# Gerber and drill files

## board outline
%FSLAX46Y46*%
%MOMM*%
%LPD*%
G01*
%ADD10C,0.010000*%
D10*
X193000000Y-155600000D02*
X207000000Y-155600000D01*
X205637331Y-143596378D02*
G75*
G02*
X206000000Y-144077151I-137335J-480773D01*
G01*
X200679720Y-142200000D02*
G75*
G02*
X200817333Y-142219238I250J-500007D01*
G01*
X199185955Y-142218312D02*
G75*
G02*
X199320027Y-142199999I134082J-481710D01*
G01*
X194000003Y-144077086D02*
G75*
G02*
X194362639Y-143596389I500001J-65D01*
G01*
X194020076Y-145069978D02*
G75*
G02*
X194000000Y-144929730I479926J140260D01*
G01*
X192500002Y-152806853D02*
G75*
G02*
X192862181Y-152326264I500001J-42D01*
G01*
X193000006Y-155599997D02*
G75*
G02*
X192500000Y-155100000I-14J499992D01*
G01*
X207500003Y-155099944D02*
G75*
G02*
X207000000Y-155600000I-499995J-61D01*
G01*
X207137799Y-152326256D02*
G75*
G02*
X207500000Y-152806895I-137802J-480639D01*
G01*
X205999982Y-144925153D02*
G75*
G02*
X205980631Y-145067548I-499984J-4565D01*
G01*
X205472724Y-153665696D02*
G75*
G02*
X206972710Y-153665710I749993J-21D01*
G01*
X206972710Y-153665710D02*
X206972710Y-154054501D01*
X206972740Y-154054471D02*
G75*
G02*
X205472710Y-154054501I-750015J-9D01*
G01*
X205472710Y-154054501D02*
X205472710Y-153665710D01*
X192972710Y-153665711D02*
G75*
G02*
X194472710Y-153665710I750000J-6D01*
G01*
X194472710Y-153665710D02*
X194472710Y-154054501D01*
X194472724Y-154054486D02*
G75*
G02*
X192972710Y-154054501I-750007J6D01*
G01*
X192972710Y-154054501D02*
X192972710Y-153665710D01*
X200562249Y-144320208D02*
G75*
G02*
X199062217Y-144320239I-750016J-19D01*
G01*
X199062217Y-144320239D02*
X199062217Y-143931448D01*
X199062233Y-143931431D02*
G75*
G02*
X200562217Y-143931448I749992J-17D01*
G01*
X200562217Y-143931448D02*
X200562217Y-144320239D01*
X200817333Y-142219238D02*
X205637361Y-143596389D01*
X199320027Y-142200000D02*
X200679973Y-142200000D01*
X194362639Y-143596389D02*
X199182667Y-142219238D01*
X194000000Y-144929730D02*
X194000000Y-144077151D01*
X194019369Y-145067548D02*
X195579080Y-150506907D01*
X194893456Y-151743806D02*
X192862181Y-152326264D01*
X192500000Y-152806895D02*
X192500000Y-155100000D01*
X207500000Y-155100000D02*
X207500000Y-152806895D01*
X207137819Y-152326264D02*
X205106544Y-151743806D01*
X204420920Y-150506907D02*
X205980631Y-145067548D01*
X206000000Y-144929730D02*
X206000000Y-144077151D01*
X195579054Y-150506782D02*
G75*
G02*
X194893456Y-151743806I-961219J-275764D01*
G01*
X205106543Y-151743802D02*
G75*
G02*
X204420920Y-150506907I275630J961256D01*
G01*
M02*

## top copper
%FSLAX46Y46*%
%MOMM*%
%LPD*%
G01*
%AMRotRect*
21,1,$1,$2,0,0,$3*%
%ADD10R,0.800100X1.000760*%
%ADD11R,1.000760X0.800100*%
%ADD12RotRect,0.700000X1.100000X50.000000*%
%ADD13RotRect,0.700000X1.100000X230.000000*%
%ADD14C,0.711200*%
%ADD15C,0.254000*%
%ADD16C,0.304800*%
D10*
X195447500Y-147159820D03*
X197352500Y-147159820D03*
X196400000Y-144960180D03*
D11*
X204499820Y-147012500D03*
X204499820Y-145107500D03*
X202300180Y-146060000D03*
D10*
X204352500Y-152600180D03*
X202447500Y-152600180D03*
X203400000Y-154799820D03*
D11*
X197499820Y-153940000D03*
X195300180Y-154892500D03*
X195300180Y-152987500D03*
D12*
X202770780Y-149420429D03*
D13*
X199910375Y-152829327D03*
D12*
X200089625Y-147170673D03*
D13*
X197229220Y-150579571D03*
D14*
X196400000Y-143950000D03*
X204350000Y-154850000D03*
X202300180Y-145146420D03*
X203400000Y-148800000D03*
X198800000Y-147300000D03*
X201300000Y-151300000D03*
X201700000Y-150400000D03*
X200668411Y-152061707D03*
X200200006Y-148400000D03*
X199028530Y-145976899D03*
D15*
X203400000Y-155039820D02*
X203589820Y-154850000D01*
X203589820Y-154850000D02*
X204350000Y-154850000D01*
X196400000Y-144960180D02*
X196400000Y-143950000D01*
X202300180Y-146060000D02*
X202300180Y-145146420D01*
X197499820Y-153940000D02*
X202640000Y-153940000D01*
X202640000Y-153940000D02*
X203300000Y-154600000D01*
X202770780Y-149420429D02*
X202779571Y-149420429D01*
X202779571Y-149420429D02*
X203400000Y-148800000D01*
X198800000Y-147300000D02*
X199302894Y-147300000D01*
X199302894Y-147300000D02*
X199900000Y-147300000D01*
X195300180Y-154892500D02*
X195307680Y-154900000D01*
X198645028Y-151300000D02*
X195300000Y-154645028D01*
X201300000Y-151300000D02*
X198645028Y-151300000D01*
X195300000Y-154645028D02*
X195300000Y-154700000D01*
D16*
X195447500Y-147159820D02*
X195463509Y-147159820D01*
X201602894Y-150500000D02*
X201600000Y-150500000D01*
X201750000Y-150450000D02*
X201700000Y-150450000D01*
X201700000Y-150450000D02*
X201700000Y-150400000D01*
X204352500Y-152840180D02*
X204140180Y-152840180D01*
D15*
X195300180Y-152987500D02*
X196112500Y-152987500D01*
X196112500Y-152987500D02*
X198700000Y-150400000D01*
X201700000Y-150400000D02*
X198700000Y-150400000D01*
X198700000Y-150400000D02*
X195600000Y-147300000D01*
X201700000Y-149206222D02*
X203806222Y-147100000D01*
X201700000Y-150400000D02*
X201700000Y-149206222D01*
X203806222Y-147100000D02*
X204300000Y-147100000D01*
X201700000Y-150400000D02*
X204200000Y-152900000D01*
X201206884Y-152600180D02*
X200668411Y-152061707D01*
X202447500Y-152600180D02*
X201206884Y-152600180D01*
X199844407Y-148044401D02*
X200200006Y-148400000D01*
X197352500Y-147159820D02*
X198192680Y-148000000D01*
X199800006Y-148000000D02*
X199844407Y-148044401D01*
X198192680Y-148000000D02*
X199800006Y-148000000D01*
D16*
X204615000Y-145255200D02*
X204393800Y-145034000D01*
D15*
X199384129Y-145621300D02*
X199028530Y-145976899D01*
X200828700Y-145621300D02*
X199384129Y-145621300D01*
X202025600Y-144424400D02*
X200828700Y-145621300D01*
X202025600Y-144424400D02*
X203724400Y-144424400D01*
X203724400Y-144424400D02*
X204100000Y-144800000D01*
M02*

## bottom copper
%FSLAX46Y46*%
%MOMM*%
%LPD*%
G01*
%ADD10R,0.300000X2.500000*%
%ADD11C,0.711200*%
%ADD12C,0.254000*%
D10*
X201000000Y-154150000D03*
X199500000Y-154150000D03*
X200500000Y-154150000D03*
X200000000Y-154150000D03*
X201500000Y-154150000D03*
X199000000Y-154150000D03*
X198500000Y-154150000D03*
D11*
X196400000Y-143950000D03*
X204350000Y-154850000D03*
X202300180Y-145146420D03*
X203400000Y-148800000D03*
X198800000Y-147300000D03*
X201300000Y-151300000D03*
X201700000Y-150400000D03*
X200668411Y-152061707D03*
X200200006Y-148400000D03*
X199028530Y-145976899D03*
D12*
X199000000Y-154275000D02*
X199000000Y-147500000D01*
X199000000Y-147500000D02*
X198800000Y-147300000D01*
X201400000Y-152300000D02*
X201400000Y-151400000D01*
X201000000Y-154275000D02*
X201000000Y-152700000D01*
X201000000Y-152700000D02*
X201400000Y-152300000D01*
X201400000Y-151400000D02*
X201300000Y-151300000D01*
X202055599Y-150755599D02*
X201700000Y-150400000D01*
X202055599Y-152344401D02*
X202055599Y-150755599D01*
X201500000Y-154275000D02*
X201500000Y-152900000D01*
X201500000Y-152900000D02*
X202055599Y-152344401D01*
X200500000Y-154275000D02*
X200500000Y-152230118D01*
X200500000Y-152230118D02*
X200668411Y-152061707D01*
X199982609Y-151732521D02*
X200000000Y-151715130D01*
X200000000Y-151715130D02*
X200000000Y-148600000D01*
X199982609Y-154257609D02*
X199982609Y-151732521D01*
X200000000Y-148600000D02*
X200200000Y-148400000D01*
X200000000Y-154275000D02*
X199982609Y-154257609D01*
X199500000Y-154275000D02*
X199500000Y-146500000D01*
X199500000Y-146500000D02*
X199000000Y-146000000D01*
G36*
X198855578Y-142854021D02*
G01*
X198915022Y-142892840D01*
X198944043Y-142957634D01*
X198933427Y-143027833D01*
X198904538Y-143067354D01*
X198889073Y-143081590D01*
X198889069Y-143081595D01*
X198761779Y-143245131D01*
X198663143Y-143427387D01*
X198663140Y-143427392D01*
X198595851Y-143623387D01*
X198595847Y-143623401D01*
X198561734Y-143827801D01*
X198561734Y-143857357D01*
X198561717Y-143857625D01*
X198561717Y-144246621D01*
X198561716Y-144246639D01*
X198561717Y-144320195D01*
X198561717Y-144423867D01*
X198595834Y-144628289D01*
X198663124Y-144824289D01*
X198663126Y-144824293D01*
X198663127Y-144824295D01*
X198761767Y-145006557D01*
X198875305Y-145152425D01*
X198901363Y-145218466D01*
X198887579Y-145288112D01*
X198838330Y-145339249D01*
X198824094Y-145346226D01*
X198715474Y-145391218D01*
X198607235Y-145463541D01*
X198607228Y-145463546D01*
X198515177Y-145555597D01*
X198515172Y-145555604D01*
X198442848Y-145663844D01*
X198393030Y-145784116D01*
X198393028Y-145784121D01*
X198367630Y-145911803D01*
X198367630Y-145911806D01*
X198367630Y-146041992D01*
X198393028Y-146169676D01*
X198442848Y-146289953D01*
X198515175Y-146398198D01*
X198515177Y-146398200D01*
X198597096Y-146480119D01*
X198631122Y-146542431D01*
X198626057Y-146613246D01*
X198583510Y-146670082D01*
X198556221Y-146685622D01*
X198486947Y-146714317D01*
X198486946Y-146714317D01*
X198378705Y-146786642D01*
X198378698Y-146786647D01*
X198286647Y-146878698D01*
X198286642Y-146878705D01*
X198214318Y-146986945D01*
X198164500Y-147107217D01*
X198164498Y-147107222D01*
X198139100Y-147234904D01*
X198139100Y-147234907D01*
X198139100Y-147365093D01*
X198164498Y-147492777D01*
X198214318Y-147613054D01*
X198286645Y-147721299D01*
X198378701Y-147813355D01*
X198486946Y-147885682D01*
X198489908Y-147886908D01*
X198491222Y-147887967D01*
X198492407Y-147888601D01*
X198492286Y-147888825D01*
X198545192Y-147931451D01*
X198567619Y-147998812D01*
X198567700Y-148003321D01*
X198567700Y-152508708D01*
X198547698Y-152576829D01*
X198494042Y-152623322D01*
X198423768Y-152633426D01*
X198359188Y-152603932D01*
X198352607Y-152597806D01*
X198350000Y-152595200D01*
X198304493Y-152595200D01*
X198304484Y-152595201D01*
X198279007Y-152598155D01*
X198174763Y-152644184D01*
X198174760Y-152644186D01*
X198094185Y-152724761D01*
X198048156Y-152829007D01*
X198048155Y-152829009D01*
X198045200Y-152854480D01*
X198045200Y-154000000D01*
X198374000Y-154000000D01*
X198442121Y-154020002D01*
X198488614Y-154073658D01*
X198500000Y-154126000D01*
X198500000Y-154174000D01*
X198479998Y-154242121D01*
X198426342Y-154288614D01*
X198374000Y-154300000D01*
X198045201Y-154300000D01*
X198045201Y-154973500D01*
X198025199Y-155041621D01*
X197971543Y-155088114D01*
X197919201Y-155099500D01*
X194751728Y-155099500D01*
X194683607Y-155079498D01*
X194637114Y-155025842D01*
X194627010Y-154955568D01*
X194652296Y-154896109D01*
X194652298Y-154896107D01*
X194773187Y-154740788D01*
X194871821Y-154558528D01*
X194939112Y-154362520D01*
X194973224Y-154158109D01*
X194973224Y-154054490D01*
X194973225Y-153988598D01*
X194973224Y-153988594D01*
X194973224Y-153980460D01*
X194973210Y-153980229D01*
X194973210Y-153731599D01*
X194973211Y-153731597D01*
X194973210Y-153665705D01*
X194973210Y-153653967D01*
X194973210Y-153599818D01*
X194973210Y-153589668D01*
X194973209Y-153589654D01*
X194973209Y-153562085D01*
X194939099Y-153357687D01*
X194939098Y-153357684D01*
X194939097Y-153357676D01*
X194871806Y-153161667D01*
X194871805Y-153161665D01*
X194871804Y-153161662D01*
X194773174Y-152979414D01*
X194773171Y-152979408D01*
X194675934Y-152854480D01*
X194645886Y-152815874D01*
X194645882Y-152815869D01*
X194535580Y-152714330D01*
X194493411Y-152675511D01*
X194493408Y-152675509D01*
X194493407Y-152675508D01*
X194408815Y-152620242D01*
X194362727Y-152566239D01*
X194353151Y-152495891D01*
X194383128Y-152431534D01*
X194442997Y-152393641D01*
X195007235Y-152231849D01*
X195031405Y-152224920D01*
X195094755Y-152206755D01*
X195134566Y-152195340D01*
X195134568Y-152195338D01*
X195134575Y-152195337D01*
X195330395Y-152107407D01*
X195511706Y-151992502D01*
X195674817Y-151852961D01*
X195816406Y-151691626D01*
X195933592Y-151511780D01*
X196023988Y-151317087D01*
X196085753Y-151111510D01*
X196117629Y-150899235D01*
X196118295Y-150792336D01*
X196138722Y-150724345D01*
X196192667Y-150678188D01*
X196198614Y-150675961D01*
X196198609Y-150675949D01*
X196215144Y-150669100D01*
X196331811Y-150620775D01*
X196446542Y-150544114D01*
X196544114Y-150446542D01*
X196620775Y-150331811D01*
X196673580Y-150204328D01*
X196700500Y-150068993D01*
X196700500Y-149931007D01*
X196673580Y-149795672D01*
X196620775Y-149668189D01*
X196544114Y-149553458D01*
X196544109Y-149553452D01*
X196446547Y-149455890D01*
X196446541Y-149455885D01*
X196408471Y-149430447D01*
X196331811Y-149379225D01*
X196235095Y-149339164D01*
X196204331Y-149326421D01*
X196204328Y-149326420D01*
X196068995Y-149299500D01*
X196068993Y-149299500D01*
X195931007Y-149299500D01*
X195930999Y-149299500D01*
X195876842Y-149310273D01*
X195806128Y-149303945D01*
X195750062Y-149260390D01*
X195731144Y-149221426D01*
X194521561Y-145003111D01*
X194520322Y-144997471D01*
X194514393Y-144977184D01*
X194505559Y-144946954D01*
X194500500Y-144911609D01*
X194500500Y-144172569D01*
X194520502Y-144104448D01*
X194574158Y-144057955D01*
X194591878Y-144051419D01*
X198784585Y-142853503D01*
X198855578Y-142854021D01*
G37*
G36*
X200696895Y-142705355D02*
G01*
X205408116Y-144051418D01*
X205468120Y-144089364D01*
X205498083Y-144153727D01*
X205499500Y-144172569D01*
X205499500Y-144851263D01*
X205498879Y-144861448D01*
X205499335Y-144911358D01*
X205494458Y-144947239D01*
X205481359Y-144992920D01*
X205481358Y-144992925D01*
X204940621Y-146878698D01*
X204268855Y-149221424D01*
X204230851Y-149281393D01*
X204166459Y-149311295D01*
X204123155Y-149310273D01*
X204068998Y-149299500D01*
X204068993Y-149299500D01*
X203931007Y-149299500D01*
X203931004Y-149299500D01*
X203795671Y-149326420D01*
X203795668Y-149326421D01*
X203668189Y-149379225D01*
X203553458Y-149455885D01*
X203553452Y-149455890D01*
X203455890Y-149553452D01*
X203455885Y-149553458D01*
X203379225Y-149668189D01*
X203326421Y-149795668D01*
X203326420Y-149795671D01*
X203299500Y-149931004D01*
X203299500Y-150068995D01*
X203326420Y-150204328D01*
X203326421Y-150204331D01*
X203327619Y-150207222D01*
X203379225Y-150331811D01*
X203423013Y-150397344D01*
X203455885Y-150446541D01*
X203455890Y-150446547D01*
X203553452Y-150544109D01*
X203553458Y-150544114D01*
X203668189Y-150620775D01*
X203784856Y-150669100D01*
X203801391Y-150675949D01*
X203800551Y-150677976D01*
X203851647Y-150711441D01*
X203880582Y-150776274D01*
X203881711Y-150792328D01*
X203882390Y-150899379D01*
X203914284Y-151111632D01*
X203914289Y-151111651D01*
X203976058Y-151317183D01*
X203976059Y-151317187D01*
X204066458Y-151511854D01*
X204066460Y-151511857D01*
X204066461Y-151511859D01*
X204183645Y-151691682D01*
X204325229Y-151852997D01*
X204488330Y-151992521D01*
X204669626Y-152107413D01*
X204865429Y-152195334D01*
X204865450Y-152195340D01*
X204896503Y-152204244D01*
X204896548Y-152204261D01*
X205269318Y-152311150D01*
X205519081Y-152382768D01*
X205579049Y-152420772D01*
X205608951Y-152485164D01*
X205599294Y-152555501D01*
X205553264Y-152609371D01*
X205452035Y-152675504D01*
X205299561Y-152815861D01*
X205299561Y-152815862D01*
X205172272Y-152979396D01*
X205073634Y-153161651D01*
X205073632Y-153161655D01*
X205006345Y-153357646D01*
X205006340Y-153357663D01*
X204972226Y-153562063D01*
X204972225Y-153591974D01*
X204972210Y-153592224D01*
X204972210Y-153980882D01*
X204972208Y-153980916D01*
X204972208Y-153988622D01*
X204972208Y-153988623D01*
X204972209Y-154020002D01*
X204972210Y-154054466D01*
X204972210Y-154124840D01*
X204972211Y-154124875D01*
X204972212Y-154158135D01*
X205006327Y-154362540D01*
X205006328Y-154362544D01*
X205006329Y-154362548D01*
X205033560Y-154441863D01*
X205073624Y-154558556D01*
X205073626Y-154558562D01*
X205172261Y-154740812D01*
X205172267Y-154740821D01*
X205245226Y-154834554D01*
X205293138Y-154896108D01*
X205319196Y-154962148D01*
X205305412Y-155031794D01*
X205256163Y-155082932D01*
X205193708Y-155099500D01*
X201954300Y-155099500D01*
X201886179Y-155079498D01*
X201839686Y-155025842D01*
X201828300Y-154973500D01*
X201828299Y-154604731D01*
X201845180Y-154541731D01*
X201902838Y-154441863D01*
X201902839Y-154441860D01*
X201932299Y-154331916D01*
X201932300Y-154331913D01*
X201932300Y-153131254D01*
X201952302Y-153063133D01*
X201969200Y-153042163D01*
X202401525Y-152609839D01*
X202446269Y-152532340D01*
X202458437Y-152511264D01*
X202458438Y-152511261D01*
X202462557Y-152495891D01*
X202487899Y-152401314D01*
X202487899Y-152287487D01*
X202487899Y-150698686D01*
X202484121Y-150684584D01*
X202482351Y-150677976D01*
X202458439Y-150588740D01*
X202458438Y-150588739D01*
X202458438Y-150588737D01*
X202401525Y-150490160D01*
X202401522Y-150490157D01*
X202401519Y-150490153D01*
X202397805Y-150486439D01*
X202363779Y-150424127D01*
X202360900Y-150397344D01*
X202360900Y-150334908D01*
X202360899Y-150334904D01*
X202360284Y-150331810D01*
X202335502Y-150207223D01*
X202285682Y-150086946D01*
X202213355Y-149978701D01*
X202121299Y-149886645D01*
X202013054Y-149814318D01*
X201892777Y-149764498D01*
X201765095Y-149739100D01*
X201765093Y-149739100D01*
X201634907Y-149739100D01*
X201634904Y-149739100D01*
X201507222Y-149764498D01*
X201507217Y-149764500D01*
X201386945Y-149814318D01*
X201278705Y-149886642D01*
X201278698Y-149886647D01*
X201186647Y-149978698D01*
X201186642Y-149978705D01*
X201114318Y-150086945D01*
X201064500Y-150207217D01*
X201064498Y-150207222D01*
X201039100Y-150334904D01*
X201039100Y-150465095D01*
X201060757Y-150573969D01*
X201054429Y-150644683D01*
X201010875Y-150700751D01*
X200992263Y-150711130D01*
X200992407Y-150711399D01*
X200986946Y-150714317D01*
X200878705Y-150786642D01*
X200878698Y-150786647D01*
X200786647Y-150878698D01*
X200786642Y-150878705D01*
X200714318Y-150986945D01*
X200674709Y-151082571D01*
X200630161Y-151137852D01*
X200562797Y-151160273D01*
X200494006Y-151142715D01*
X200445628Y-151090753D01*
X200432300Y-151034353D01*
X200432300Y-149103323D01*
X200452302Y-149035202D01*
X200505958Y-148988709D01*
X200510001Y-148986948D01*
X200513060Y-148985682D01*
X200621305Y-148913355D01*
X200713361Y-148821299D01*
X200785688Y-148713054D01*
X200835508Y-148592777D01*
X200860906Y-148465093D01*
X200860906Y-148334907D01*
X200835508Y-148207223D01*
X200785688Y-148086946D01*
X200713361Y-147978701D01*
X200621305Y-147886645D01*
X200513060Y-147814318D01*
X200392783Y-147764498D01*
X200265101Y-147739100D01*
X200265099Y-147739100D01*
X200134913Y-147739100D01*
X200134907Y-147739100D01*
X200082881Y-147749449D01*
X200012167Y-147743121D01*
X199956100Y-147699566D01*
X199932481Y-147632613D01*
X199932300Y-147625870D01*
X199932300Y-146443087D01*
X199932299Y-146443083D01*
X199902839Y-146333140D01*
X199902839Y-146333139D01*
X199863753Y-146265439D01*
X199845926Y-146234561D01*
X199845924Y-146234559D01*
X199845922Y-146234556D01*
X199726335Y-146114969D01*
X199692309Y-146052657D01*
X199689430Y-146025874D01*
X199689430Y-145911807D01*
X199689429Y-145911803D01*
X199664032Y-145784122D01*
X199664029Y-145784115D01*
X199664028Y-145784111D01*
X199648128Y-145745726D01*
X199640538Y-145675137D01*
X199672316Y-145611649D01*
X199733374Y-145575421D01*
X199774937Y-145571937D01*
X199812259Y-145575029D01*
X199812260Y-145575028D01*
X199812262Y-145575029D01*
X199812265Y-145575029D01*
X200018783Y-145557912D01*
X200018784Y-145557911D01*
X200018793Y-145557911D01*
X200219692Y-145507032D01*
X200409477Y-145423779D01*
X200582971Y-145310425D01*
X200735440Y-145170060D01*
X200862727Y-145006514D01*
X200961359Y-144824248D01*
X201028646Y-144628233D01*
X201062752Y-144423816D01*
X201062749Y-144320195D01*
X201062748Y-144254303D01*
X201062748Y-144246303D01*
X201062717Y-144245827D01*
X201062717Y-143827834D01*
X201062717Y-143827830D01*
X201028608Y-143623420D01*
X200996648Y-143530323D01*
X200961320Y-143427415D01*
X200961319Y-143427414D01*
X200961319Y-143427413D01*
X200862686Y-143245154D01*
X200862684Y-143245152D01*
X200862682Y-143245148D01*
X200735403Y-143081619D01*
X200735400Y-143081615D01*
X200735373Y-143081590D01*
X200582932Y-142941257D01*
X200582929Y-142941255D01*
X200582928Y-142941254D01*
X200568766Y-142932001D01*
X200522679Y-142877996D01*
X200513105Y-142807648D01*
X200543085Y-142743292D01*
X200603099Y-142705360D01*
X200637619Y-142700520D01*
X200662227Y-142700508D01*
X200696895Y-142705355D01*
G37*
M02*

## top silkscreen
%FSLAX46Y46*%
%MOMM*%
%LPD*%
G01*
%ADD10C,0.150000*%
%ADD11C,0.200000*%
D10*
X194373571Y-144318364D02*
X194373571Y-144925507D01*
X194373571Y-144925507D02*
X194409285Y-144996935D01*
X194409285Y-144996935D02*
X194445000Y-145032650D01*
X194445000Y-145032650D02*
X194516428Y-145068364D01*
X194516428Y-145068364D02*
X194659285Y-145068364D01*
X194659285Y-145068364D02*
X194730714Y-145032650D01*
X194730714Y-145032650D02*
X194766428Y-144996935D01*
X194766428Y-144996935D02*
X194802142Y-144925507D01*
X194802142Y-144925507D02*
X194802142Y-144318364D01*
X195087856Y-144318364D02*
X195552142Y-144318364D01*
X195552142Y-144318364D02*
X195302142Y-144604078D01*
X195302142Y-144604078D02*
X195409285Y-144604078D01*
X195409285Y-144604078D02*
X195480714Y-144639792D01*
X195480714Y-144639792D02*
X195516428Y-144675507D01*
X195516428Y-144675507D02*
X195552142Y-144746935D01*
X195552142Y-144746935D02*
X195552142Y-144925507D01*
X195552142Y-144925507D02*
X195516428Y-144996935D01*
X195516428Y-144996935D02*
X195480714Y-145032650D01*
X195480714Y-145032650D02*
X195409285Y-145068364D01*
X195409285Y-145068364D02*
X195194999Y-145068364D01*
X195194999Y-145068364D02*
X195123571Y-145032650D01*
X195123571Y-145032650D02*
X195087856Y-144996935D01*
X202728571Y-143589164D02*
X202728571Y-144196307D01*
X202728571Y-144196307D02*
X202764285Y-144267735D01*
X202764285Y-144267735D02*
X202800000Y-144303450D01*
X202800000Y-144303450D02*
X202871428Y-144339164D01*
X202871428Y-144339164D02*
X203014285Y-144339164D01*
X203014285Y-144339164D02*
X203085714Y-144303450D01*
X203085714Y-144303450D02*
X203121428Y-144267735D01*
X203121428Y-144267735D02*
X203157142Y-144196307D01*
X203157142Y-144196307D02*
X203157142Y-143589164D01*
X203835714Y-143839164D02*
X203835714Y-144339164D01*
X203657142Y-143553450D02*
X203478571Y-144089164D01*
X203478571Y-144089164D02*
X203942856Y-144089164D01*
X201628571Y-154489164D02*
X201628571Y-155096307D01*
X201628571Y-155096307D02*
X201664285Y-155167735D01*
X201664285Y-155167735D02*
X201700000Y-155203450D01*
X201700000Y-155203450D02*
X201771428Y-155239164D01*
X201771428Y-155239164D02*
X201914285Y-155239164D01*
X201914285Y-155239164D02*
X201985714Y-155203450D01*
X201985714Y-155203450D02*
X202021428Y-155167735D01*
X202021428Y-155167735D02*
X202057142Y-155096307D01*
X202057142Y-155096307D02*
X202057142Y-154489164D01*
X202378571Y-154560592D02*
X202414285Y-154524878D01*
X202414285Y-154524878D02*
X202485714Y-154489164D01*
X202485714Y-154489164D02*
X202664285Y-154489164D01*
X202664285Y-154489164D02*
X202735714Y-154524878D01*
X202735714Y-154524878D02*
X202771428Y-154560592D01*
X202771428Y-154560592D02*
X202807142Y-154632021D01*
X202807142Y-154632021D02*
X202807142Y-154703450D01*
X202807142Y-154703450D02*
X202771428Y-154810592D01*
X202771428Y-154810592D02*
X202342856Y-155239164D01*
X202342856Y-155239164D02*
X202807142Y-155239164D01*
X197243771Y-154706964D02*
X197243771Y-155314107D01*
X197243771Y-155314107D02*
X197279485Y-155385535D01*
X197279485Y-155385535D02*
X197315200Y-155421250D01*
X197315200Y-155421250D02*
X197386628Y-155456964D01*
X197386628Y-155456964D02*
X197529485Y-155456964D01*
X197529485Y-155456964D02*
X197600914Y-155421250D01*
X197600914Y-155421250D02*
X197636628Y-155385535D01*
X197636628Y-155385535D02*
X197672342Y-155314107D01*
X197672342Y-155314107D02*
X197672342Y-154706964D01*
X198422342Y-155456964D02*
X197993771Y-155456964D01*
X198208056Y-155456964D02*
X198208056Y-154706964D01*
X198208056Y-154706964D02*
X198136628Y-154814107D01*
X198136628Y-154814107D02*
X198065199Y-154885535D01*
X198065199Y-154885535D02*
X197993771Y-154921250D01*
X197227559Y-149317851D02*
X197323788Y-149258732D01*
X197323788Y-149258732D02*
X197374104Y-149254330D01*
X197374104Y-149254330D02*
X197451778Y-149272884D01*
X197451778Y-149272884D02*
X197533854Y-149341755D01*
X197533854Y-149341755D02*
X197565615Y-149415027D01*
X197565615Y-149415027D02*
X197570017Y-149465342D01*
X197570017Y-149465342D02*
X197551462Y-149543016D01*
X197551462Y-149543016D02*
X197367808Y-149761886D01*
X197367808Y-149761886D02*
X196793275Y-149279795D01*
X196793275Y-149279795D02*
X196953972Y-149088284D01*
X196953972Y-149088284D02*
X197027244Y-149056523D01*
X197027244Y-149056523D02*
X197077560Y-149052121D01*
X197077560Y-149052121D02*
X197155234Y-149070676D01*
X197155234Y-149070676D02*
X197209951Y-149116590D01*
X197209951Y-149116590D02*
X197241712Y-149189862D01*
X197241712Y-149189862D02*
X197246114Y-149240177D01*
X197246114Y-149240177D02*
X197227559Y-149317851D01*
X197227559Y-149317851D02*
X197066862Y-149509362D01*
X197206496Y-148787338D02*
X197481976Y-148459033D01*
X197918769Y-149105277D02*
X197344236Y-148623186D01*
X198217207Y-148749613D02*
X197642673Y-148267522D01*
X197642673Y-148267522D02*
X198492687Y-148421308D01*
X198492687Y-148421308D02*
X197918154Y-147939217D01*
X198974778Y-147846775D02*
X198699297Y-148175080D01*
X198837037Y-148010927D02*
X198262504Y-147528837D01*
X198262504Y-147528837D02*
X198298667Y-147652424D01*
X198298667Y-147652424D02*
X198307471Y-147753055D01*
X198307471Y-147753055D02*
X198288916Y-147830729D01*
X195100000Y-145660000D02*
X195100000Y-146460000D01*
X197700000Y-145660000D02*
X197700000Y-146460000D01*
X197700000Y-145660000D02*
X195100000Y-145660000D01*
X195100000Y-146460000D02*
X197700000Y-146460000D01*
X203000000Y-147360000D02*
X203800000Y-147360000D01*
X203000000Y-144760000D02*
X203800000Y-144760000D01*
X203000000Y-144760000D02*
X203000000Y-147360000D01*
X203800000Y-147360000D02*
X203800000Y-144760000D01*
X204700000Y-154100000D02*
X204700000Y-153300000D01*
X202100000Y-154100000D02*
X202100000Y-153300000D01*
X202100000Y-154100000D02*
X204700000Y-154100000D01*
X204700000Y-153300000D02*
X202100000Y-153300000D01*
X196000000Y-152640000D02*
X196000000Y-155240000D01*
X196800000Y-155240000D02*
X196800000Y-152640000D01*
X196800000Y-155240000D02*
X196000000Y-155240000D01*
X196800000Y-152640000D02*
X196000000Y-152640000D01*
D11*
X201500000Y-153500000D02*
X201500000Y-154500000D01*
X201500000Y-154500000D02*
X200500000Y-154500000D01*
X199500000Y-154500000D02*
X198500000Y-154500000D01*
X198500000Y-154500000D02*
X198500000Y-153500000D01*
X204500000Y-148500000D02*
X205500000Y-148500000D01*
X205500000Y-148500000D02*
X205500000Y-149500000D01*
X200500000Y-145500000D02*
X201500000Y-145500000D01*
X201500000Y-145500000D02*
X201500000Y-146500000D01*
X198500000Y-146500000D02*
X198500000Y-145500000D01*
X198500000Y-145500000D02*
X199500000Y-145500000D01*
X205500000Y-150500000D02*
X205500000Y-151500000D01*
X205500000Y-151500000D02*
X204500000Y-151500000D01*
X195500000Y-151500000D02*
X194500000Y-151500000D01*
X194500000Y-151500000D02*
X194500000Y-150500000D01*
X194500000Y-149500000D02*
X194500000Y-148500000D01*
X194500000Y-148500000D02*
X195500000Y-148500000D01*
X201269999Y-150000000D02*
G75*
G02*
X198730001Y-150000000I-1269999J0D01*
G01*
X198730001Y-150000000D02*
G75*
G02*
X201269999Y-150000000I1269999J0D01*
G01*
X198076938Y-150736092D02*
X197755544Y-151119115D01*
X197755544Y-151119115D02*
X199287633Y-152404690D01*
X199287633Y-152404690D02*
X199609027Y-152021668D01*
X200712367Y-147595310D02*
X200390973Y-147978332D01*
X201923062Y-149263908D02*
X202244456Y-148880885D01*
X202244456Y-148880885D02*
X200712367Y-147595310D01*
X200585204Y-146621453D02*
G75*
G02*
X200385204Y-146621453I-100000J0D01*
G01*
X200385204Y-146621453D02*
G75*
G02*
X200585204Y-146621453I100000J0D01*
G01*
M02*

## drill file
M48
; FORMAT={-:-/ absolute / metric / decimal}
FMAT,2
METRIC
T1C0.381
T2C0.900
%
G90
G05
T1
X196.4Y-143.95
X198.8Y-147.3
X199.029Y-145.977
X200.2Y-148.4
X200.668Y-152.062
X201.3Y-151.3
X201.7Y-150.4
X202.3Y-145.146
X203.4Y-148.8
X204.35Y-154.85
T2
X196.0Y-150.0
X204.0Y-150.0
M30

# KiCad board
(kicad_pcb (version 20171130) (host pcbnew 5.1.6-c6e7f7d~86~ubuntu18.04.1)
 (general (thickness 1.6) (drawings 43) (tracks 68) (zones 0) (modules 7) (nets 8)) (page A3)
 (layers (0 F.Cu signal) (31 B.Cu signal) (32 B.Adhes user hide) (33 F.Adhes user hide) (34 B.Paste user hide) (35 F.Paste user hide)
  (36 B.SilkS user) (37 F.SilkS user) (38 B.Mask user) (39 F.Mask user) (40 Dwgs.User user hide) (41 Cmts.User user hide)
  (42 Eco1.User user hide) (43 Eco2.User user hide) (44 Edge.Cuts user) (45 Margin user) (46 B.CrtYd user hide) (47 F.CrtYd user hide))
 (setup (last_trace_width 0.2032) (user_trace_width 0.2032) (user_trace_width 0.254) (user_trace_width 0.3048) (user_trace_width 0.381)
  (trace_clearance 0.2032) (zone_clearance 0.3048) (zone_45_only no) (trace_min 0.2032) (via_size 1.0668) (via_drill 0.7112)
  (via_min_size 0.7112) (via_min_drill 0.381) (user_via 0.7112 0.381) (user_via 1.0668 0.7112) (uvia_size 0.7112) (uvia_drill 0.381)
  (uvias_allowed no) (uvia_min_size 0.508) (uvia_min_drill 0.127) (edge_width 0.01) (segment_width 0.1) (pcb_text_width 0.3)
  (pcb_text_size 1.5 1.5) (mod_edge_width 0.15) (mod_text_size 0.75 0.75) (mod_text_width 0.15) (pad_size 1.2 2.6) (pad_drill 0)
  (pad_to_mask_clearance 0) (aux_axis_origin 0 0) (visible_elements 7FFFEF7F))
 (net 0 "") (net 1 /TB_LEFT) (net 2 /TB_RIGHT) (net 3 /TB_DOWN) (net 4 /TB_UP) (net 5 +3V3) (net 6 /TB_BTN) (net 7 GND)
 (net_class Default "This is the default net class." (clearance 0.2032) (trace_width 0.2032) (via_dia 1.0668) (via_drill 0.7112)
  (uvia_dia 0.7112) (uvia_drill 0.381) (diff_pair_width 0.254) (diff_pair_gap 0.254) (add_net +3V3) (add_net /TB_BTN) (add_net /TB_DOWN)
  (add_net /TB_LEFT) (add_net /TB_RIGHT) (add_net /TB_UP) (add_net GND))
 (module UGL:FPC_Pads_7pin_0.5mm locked (layer B.Cu) (at 200 155.4 180)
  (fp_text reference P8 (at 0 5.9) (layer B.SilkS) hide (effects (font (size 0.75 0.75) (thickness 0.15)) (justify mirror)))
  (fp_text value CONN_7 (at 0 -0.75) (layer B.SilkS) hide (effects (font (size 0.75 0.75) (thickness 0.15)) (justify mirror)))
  (pad 2 smd rect (at -1 1.25 180) (size 0.3 2.5) (layers B.Cu B.Mask) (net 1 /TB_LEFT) (clearance 0.1778))
  (pad 5 smd rect (at 0.5 1.25 180) (size 0.3 2.5) (layers B.Cu B.Mask) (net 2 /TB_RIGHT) (clearance 0.1778))
  (pad 3 smd rect (at -0.5 1.25 180) (size 0.3 2.5) (layers B.Cu B.Mask) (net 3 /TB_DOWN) (clearance 0.1778))
  (pad 4 smd rect (at 0 1.25 180) (size 0.3 2.5) (layers B.Cu B.Mask) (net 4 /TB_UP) (clearance 0.1778))
  (pad 1 smd rect (at -1.5 1.25 180) (size 0.3 2.5) (layers B.Cu B.Mask) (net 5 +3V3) (clearance 0.1778))
  (pad 6 smd rect (at 1 1.25 180) (size 0.3 2.5) (layers B.Cu B.Mask) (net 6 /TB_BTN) (clearance 0.1778))
  (pad 7 smd rect (at 1.5 1.25 180) (size 0.3 2.5) (layers B.Cu B.Mask) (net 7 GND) (clearance 0.1778)))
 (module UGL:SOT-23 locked (layer F.Cu) (at 196.4 146.06)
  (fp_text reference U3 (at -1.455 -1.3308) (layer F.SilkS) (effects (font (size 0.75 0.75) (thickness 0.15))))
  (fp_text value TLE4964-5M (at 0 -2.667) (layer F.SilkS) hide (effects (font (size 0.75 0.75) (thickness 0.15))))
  (fp_line (start -1.3 -0.4) (end -1.3 0.4) (layer F.SilkS) (width 0.15))
  (fp_line (start 1.3 -0.4) (end 1.3 0.4) (layer F.SilkS) (width 0.15))
  (fp_line (start 1.3 -0.4) (end -1.3 -0.4) (layer F.SilkS) (width 0.15))
  (fp_line (start -1.3 0.4) (end 1.3 0.4) (layer F.SilkS) (width 0.15))
  (pad 1 smd rect (at -0.9525 1.09982) (size 0.8001 1.00076) (layers F.Cu F.Paste F.Mask) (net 5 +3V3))
  (pad 2 smd rect (at 0.9525 1.09982) (size 0.8001 1.00076) (layers F.Cu F.Paste F.Mask) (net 4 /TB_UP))
  (pad 3 smd rect (at 0 -1.09982) (size 0.8001 1.00076) (layers F.Cu F.Paste F.Mask) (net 7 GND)))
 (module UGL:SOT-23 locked (layer F.Cu) (at 203.4 146.06 90)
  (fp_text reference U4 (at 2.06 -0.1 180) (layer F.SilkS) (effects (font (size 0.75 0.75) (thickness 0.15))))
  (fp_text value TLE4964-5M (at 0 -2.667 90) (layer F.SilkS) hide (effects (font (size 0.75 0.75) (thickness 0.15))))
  (fp_line (start -1.3 -0.4) (end -1.3 0.4) (layer F.SilkS) (width 0.15))
  (fp_line (start 1.3 -0.4) (end 1.3 0.4) (layer F.SilkS) (width 0.15))
  (fp_line (start 1.3 -0.4) (end -1.3 -0.4) (layer F.SilkS) (width 0.15))
  (fp_line (start -1.3 0.4) (end 1.3 0.4) (layer F.SilkS) (width 0.15))
  (pad 1 smd rect (at -0.9525 1.09982 90) (size 0.8001 1.00076) (layers F.Cu F.Paste F.Mask) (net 5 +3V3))
  (pad 2 smd rect (at 0.9525 1.09982 90) (size 0.8001 1.00076) (layers F.Cu F.Paste F.Mask) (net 2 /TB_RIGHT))
  (pad 3 smd rect (at 0 -1.09982 90) (size 0.8001 1.00076) (layers F.Cu F.Paste F.Mask) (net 7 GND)))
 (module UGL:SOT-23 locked (layer F.Cu) (at 203.4 153.7 180)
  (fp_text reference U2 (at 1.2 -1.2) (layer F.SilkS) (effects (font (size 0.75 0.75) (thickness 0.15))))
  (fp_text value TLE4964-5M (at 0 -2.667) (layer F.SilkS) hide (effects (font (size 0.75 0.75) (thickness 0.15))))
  (fp_line (start -1.3 -0.4) (end -1.3 0.4) (layer F.SilkS) (width 0.15))
  (fp_line (start 1.3 -0.4) (end 1.3 0.4) (layer F.SilkS) (width 0.15))
  (fp_line (start 1.3 -0.4) (end -1.3 -0.4) (layer F.SilkS) (width 0.15))
  (fp_line (start -1.3 0.4) (end 1.3 0.4) (layer F.SilkS) (width 0.15))
  (pad 1 smd rect (at -0.9525 1.09982 180) (size 0.8001 1.00076) (layers F.Cu F.Paste F.Mask) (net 5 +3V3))
  (pad 2 smd rect (at 0.9525 1.09982 180) (size 0.8001 1.00076) (layers F.Cu F.Paste F.Mask) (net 3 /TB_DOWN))
  (pad 3 smd rect (at 0 -1.09982 180) (size 0.8001 1.00076) (layers F.Cu F.Paste F.Mask) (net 7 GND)))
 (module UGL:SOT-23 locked (layer F.Cu) (at 196.4 153.94 270)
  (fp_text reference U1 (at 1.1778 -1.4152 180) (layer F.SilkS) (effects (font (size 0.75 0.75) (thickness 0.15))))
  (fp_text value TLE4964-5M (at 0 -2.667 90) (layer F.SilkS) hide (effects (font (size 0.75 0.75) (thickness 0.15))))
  (fp_line (start -1.3 0.4) (end 1.3 0.4) (layer F.SilkS) (width 0.15))
  (fp_line (start 1.3 -0.4) (end -1.3 -0.4) (layer F.SilkS) (width 0.15))
  (fp_line (start 1.3 -0.4) (end 1.3 0.4) (layer F.SilkS) (width 0.15))
  (fp_line (start -1.3 -0.4) (end -1.3 0.4) (layer F.SilkS) (width 0.15))
  (pad 3 smd rect (at 0 -1.09982 270) (size 0.8001 1.00076) (layers F.Cu F.Paste F.Mask) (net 7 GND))
  (pad 2 smd rect (at 0.9525 1.09982 270) (size 0.8001 1.00076) (layers F.Cu F.Paste F.Mask) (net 1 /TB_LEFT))
  (pad 1 smd rect (at -0.9525 1.09982 270) (size 0.8001 1.00076) (layers F.Cu F.Paste F.Mask) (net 5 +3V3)))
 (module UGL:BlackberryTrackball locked (layer F.Cu) (at 200 150)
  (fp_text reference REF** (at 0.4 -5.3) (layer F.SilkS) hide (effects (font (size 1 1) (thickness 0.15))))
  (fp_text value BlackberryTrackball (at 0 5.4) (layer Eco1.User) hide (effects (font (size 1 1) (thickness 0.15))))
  (fp_line (start 1.5 3.5) (end 1.5 4.5) (layer F.SilkS) (width 0.2))
  (fp_line (start 1.5 4.5) (end 0.5 4.5) (layer F.SilkS) (width 0.2))
  (fp_line (start -0.5 4.5) (end -1.5 4.5) (layer F.SilkS) (width 0.2))
  (fp_line (start -1.5 4.5) (end -1.5 3.5) (layer F.SilkS) (width 0.2))
  (fp_line (start 4.5 -1.5) (end 5.5 -1.5) (layer F.SilkS) (width 0.2))
  (fp_line (start 5.5 -1.5) (end 5.5 -0.5) (layer F.SilkS) (width 0.2))
  (fp_line (start 0.5 -4.5) (end 1.5 -4.5) (layer F.SilkS) (width 0.2))
  (fp_line (start 1.5 -4.5) (end 1.5 -3.5) (layer F.SilkS) (width 0.2))
  (fp_line (start -1.5 -3.5) (end -1.5 -4.5) (layer F.SilkS) (width 0.2))
  (fp_line (start -1.5 -4.5) (end -0.5 -4.5) (layer F.SilkS) (width 0.2))
  (fp_line (start 5.5 0.5) (end 5.5 1.5) (layer F.SilkS) (width 0.2))
  (fp_line (start 5.5 1.5) (end 4.5 1.5) (layer F.SilkS) (width 0.2))
  (fp_line (start -4.5 1.5) (end -5.5 1.5) (layer F.SilkS) (width 0.2))
  (fp_line (start -5.5 1.5) (end -5.5 0.5) (layer F.SilkS) (width 0.2))
  (fp_line (start -5.5 -0.5) (end -5.5 -1.5) (layer F.SilkS) (width 0.2))
  (fp_line (start -5.5 -1.5) (end -4.5 -1.5) (layer F.SilkS) (width 0.2))
  (pad "" np_thru_hole circle (at 4 0) (size 0.9 0.9) (drill 0.9) (layers *.Cu *.Mask))
  (pad "" np_thru_hole circle (at -4 0) (size 0.9 0.9) (drill 0.9) (layers *.Cu *.Mask)))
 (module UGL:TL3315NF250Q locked (layer F.Cu) (at 200 150 50)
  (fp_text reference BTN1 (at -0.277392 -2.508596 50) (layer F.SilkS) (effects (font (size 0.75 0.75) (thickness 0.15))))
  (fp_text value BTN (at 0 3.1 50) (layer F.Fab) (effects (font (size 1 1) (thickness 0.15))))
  (fp_circle (center 0 0) (end 1.27 0) (layer F.SilkS) (width 0.2))
  (fp_line (start -1.8 -1) (end -2.3 -1) (layer F.SilkS) (width 0.2))
  (fp_line (start -2.3 -1) (end -2.3 1) (layer F.SilkS) (width 0.2))
  (fp_line (start -2.3 1) (end -1.8 1) (layer F.SilkS) (width 0.2))
  (fp_line (start 2.3 -1) (end 1.8 -1) (layer F.SilkS) (width 0.2))
  (fp_line (start 1.8 1) (end 2.3 1) (layer F.SilkS) (width 0.2))
  (fp_line (start 2.3 1) (end 2.3 -1) (layer F.SilkS) (width 0.2))
  (fp_circle (center 2.9 -1.8) (end 3 -1.8) (layer F.SilkS) (width 0.2))
  (pad 2 smd rect (at 2.225 1.75 50) (size 0.7 1.1) (layers F.Cu F.Paste F.Mask) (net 7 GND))
  (pad 3 smd rect (at -2.225 1.75 230) (size 0.7 1.1) (layers F.Cu F.Paste F.Mask))
  (pad 1 smd rect (at 2.225 -1.75 50) (size 0.7 1.1) (layers F.Cu F.Paste F.Mask) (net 6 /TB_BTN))
  (pad 4 smd rect (at -2.225 -1.75 230) (size 0.7 1.1) (layers F.Cu F.Paste F.Mask)))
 (gr_line (start 193 155.6) (end 207 155.6) (angle 90) (layer Edge.Cuts) (width 0.01))
 (gr_arc (start 205.499996 144.077151) (end 206 144.077151) (angle -74.05780781) (layer Edge.Cuts) (width 0.01))
 (gr_arc (start 200.67997 142.700007) (end 200.817333 142.219238) (angle -15.97405795) (layer Edge.Cuts) (width 0.01))
 (gr_arc (start 199.320037 142.700022) (end 199.320027 142.2) (angle -15.55315467) (layer Edge.Cuts) (width 0.01))
 (gr_arc (start 194.500004 144.077151) (end 194.362639 143.596389) (angle -74.04666612) (layer Edge.Cuts) (width 0.01))
 (gr_arc (start 194.500002 144.929718) (end 194 144.92973) (angle -16.28978266) (layer Edge.Cuts) (width 0.01))
 (gr_arc (start 193.000003 152.806895) (end 192.862181 152.326264) (angle -73.99483282) (layer Edge.Cuts) (width 0.01))
 (gr_arc (start 192.999992 155.100005) (end 192.5 155.1) (angle -90.00219193) (layer Edge.Cuts) (width 0.01))
 (gr_arc (start 207.000008 155.100005) (end 207 155.6) (angle -90.00795646) (layer Edge.Cuts) (width 0.01))
 (gr_arc (start 206.999997 152.806895) (end 207.5 152.806895) (angle -74.00205761) (layer Edge.Cuts) (width 0.01))
 (gr_arc (start 205.499998 144.929718) (end 205.980631 145.067548) (angle -16.5242857) (layer Edge.Cuts) (width 0.01))
 (gr_arc (start 206.222717 153.665717) (end 206.97271 153.66571) (angle -179.9978282) (layer Edge.Cuts) (width 0.01))
 (gr_line (start 206.97271 153.66571) (end 206.97271 154.054501) (angle 90) (layer Edge.Cuts) (width 0.01))
 (gr_arc (start 206.222725 154.05448) (end 205.47271 154.054501) (angle -179.9990721) (layer Edge.Cuts) (width 0.01))
 (gr_line (start 205.47271 154.054501) (end 205.47271 153.66571) (angle 90) (layer Edge.Cuts) (width 0.01))
 (gr_arc (start 193.72271 153.665717) (end 194.47271 153.66571) (angle -179.9989939) (layer Edge.Cuts) (width 0.01))
 (gr_line (start 194.47271 153.66571) (end 194.47271 154.054501) (angle 90) (layer Edge.Cuts) (width 0.01))
 (gr_arc (start 193.722717 154.05448) (end 192.97271 154.054501) (angle -179.9979064) (layer Edge.Cuts) (width 0.01))
 (gr_line (start 192.97271 154.054501) (end 192.97271 153.66571) (angle 90) (layer Edge.Cuts) (width 0.01))
 (gr_arc (start 199.812233 144.320227) (end 199.062217 144.320239) (angle -180.0005206) (layer Edge.Cuts) (width 0.01))
 (gr_line (start 199.062217 144.320239) (end 199.062217 143.931448) (angle 90) (layer Edge.Cuts) (width 0.01))
 (gr_arc (start 199.812225 143.931448) (end 200.562217 143.931448) (angle -179.9987111) (layer Edge.Cuts) (width 0.01))
 (gr_line (start 200.562217 143.931448) (end 200.562217 144.320239) (angle 90) (layer Edge.Cuts) (width 0.01))
 (gr_line (start 200.817333 142.219238) (end 205.637361 143.596389) (angle 90) (layer Edge.Cuts) (width 0.01))
 (gr_line (start 199.320027 142.2) (end 200.679973 142.2) (angle 90) (layer Edge.Cuts) (width 0.01))
 (gr_line (start 194.362639 143.596389) (end 199.182667 142.219238) (angle 90) (layer Edge.Cuts) (width 0.01))
 (gr_line (start 194 144.92973) (end 194 144.077151) (angle 90) (layer Edge.Cuts) (width 0.01))
 (gr_line (start 194.019369 145.067548) (end 195.57908 150.506907) (angle 90) (layer Edge.Cuts) (width 0.01))
 (gr_line (start 194.893456 151.743806) (end 192.862181 152.326264) (angle 90) (layer Edge.Cuts) (width 0.01))
 (gr_line (start 192.5 152.806895) (end 192.5 155.1) (angle 90) (layer Edge.Cuts) (width 0.01))
 (gr_line (start 207.5 155.1) (end 207.5 152.806895) (angle 90) (layer Edge.Cuts) (width 0.01))
 (gr_line (start 207.137819 152.326264) (end 205.106544 151.743806) (angle 90) (layer Edge.Cuts) (width 0.01))
 (gr_line (start 204.42092 150.506907) (end 205.980631 145.067548) (angle 90) (layer Edge.Cuts) (width 0.01))
 (gr_line (start 206 144.92973) (end 206 144.077151) (angle 90) (layer Edge.Cuts) (width 0.01))
 (gr_arc (start 194.617835 150.782546) (end 194.893456 151.743806) (angle -90.00852698) (layer Edge.Cuts) (width 0.01))
 (gr_arc (start 205.382173 150.782546) (end 204.42092 150.506907) (angle -90.00052091) (layer Edge.Cuts) (width 0.01))
 (via (at 196.4 143.95) (size 0.7112) (drill 0.381) (layers F.Cu B.Cu) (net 7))
 (segment (start 203.4 155.03982) (end 203.58982 154.85) (width 0.254) (layer F.Cu) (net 7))
 (via (at 204.35 154.85) (size 0.7112) (drill 0.381) (layers F.Cu B.Cu) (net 7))
 (segment (start 203.58982 154.85) (end 204.35 154.85) (width 0.254) (layer F.Cu) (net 7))
 (segment (start 196.4 144.96018) (end 196.4 143.95) (width 0.254) (layer F.Cu) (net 7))
 (segment (start 202.30018 146.06) (end 202.30018 145.14642) (width 0.254) (layer F.Cu) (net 7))
 (via (at 202.30018 145.14642) (size 0.7112) (drill 0.381) (layers F.Cu B.Cu) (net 7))
 (segment (start 197.49982 153.94) (end 202.64 153.94) (width 0.254) (layer F.Cu) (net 7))
 (segment (start 202.64 153.94) (end 203.3 154.6) (width 0.254) (layer F.Cu) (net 7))
 (via (at 203.4 148.8) (size 0.7112) (drill 0.381) (layers F.Cu B.Cu) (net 7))
 (segment (start 202.77078 149.420429) (end 202.779571 149.420429) (width 0.254) (layer F.Cu) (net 7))
 (segment (start 202.779571 149.420429) (end 203.4 148.8) (width 0.254) (layer F.Cu) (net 7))
 (via (at 198.8 147.3) (size 0.7112) (drill 0.381) (layers F.Cu B.Cu) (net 6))
 (segment (start 198.8 147.3) (end 199.302894 147.3) (width 0.254) (layer F.Cu) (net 6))
 (segment (start 199.302894 147.3) (end 199.9 147.3) (width 0.254) (layer F.Cu) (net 6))
 (segment (start 199 154.275) (end 199 147.5) (width 0.254) (layer B.Cu) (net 6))
 (segment (start 199 147.5) (end 198.8 147.3) (width 0.254) (layer B.Cu) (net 6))
 (segment (start 195.30018 154.8925) (end 195.30768 154.9) (width 0.254) (layer F.Cu) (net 1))
 (via (at 201.3 151.3) (size 0.7112) (drill 0.381) (layers F.Cu B.Cu) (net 1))
 (segment (start 198.645028 151.3) (end 195.3 154.645028) (width 0.254) (layer F.Cu) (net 1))
 (segment (start 201.3 151.3) (end 198.645028 151.3) (width 0.254) (layer F.Cu) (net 1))
 (segment (start 195.3 154.645028) (end 195.3 154.7) (width 0.254) (layer F.Cu) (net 1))
 (segment (start 201.4 152.3) (end 201.4 151.4) (width 0.254) (layer B.Cu) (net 1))
 (segment (start 201 154.275) (end 201 152.7) (width 0.254) (layer B.Cu) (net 1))
 (segment (start 201 152.7) (end 201.4 152.3) (width 0.254) (layer B.Cu) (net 1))
 (segment (start 201.4 151.4) (end 201.3 151.3) (width 0.254) (layer B.Cu) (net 1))
 (segment (start 195.4475 147.15982) (end 195.463509 147.15982) (width 0.3048) (layer F.Cu) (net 5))
 (segment (start 201.602894 150.5) (end 201.6 150.5) (width 0.3048) (layer F.Cu) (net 5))
 (via (at 201.7 150.4) (size 0.7112) (drill 0.381) (layers F.Cu B.Cu) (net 5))
 (segment (start 201.75 150.45) (end 201.7 150.45) (width 0.3048) (layer F.Cu) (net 5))
 (segment (start 201.7 150.45) (end 201.7 150.4) (width 0.3048) (layer F.Cu) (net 5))
 (segment (start 204.3525 152.84018) (end 204.14018 152.84018) (width 0.3048) (layer F.Cu) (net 5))
 (segment (start 195.30018 152.9875) (end 196.1125 152.9875) (width 0.254) (layer F.Cu) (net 5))
 (segment (start 196.1125 152.9875) (end 198.7 150.4) (width 0.254) (layer F.Cu) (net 5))
 (segment (start 201.7 150.4) (end 198.7 150.4) (width 0.254) (layer F.Cu) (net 5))
 (segment (start 198.7 150.4) (end 195.6 147.3) (width 0.254) (layer F.Cu) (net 5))
 (segment (start 201.7 149.206222) (end 203.806222 147.1) (width 0.254) (layer F.Cu) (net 5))
 (segment (start 201.7 150.4) (end 201.7 149.206222) (width 0.254) (layer F.Cu) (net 5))
 (segment (start 203.806222 147.1) (end 204.3 147.1) (width 0.254) (layer F.Cu) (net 5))
 (segment (start 201.7 150.4) (end 204.2 152.9) (width 0.254) (layer F.Cu) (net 5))
 (segment (start 202.055599 150.755599) (end 201.7 150.4) (width 0.254) (layer B.Cu) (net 5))
 (segment (start 202.055599 152.344401) (end 202.055599 150.755599) (width 0.254) (layer B.Cu) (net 5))
 (segment (start 201.5 154.275) (end 201.5 152.9) (width 0.254) (layer B.Cu) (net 5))
 (segment (start 201.5 152.9) (end 202.055599 152.344401) (width 0.254) (layer B.Cu) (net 5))
 (via (at 200.668411 152.061707) (size 0.7112) (drill 0.381) (layers F.Cu B.Cu) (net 3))
 (segment (start 201.206884 152.60018) (end 200.668411 152.061707) (width 0.254) (layer F.Cu) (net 3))
 (segment (start 202.4475 152.60018) (end 201.206884 152.60018) (width 0.254) (layer F.Cu) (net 3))
 (segment (start 200.5 154.275) (end 200.5 152.230118) (width 0.254) (layer B.Cu) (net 3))
 (segment (start 200.5 152.230118) (end 200.668411 152.061707) (width 0.254) (layer B.Cu) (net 3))
 (via (at 200.200006 148.4) (size 0.7112) (drill 0.381) (layers F.Cu B.Cu) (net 4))
 (segment (start 199.844407 148.044401) (end 200.200006 148.4) (width 0.254) (layer F.Cu) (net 4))
 (segment (start 197.3525 147.15982) (end 198.19268 148) (width 0.254) (layer F.Cu) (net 4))
 (segment (start 199.800006 148) (end 199.844407 148.044401) (width 0.254) (layer F.Cu) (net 4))
 (segment (start 198.19268 148) (end 199.800006 148) (width 0.254) (layer F.Cu) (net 4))
 (segment (start 199.982609 151.732521) (end 200 151.71513) (width 0.254) (layer B.Cu) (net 4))
 (segment (start 200 151.71513) (end 200 148.6) (width 0.254) (layer B.Cu) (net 4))
 (segment (start 199.982609 154.257609) (end 199.982609 151.732521) (width 0.254) (layer B.Cu) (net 4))
 (segment (start 200 148.6) (end 200.2 148.4) (width 0.254) (layer B.Cu) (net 4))
 (segment (start 200 154.275) (end 199.982609 154.257609) (width 0.254) (layer B.Cu) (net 4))
 (segment (start 204.615 145.2552) (end 204.3938 145.034) (width 0.3048) (layer F.Cu) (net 2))
 (via (at 199.02853 145.976899) (size 0.7112) (drill 0.381) (layers F.Cu B.Cu) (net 2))
 (segment (start 199.384129 145.6213) (end 199.02853 145.976899) (width 0.254) (layer F.Cu) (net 2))
 (segment (start 200.8287 145.6213) (end 199.384129 145.6213) (width 0.254) (layer F.Cu) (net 2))
 (segment (start 202.0256 144.4244) (end 200.8287 145.6213) (width 0.254) (layer F.Cu) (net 2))
 (segment (start 202.0256 144.4244) (end 203.7244 144.4244) (width 0.254) (layer F.Cu) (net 2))
 (segment (start 203.7244 144.4244) (end 204.1 144.8) (width 0.254) (layer F.Cu) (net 2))
 (segment (start 199.5 154.275) (end 199.5 146.5) (width 0.254) (layer B.Cu) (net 2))
 (segment (start 199.5 146.5) (end 199 146) (width 0.254) (layer B.Cu) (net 2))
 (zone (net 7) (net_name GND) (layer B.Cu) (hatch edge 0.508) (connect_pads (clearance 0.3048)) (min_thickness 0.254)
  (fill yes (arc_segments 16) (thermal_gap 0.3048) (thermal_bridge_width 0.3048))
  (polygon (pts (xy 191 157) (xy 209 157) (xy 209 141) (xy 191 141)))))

